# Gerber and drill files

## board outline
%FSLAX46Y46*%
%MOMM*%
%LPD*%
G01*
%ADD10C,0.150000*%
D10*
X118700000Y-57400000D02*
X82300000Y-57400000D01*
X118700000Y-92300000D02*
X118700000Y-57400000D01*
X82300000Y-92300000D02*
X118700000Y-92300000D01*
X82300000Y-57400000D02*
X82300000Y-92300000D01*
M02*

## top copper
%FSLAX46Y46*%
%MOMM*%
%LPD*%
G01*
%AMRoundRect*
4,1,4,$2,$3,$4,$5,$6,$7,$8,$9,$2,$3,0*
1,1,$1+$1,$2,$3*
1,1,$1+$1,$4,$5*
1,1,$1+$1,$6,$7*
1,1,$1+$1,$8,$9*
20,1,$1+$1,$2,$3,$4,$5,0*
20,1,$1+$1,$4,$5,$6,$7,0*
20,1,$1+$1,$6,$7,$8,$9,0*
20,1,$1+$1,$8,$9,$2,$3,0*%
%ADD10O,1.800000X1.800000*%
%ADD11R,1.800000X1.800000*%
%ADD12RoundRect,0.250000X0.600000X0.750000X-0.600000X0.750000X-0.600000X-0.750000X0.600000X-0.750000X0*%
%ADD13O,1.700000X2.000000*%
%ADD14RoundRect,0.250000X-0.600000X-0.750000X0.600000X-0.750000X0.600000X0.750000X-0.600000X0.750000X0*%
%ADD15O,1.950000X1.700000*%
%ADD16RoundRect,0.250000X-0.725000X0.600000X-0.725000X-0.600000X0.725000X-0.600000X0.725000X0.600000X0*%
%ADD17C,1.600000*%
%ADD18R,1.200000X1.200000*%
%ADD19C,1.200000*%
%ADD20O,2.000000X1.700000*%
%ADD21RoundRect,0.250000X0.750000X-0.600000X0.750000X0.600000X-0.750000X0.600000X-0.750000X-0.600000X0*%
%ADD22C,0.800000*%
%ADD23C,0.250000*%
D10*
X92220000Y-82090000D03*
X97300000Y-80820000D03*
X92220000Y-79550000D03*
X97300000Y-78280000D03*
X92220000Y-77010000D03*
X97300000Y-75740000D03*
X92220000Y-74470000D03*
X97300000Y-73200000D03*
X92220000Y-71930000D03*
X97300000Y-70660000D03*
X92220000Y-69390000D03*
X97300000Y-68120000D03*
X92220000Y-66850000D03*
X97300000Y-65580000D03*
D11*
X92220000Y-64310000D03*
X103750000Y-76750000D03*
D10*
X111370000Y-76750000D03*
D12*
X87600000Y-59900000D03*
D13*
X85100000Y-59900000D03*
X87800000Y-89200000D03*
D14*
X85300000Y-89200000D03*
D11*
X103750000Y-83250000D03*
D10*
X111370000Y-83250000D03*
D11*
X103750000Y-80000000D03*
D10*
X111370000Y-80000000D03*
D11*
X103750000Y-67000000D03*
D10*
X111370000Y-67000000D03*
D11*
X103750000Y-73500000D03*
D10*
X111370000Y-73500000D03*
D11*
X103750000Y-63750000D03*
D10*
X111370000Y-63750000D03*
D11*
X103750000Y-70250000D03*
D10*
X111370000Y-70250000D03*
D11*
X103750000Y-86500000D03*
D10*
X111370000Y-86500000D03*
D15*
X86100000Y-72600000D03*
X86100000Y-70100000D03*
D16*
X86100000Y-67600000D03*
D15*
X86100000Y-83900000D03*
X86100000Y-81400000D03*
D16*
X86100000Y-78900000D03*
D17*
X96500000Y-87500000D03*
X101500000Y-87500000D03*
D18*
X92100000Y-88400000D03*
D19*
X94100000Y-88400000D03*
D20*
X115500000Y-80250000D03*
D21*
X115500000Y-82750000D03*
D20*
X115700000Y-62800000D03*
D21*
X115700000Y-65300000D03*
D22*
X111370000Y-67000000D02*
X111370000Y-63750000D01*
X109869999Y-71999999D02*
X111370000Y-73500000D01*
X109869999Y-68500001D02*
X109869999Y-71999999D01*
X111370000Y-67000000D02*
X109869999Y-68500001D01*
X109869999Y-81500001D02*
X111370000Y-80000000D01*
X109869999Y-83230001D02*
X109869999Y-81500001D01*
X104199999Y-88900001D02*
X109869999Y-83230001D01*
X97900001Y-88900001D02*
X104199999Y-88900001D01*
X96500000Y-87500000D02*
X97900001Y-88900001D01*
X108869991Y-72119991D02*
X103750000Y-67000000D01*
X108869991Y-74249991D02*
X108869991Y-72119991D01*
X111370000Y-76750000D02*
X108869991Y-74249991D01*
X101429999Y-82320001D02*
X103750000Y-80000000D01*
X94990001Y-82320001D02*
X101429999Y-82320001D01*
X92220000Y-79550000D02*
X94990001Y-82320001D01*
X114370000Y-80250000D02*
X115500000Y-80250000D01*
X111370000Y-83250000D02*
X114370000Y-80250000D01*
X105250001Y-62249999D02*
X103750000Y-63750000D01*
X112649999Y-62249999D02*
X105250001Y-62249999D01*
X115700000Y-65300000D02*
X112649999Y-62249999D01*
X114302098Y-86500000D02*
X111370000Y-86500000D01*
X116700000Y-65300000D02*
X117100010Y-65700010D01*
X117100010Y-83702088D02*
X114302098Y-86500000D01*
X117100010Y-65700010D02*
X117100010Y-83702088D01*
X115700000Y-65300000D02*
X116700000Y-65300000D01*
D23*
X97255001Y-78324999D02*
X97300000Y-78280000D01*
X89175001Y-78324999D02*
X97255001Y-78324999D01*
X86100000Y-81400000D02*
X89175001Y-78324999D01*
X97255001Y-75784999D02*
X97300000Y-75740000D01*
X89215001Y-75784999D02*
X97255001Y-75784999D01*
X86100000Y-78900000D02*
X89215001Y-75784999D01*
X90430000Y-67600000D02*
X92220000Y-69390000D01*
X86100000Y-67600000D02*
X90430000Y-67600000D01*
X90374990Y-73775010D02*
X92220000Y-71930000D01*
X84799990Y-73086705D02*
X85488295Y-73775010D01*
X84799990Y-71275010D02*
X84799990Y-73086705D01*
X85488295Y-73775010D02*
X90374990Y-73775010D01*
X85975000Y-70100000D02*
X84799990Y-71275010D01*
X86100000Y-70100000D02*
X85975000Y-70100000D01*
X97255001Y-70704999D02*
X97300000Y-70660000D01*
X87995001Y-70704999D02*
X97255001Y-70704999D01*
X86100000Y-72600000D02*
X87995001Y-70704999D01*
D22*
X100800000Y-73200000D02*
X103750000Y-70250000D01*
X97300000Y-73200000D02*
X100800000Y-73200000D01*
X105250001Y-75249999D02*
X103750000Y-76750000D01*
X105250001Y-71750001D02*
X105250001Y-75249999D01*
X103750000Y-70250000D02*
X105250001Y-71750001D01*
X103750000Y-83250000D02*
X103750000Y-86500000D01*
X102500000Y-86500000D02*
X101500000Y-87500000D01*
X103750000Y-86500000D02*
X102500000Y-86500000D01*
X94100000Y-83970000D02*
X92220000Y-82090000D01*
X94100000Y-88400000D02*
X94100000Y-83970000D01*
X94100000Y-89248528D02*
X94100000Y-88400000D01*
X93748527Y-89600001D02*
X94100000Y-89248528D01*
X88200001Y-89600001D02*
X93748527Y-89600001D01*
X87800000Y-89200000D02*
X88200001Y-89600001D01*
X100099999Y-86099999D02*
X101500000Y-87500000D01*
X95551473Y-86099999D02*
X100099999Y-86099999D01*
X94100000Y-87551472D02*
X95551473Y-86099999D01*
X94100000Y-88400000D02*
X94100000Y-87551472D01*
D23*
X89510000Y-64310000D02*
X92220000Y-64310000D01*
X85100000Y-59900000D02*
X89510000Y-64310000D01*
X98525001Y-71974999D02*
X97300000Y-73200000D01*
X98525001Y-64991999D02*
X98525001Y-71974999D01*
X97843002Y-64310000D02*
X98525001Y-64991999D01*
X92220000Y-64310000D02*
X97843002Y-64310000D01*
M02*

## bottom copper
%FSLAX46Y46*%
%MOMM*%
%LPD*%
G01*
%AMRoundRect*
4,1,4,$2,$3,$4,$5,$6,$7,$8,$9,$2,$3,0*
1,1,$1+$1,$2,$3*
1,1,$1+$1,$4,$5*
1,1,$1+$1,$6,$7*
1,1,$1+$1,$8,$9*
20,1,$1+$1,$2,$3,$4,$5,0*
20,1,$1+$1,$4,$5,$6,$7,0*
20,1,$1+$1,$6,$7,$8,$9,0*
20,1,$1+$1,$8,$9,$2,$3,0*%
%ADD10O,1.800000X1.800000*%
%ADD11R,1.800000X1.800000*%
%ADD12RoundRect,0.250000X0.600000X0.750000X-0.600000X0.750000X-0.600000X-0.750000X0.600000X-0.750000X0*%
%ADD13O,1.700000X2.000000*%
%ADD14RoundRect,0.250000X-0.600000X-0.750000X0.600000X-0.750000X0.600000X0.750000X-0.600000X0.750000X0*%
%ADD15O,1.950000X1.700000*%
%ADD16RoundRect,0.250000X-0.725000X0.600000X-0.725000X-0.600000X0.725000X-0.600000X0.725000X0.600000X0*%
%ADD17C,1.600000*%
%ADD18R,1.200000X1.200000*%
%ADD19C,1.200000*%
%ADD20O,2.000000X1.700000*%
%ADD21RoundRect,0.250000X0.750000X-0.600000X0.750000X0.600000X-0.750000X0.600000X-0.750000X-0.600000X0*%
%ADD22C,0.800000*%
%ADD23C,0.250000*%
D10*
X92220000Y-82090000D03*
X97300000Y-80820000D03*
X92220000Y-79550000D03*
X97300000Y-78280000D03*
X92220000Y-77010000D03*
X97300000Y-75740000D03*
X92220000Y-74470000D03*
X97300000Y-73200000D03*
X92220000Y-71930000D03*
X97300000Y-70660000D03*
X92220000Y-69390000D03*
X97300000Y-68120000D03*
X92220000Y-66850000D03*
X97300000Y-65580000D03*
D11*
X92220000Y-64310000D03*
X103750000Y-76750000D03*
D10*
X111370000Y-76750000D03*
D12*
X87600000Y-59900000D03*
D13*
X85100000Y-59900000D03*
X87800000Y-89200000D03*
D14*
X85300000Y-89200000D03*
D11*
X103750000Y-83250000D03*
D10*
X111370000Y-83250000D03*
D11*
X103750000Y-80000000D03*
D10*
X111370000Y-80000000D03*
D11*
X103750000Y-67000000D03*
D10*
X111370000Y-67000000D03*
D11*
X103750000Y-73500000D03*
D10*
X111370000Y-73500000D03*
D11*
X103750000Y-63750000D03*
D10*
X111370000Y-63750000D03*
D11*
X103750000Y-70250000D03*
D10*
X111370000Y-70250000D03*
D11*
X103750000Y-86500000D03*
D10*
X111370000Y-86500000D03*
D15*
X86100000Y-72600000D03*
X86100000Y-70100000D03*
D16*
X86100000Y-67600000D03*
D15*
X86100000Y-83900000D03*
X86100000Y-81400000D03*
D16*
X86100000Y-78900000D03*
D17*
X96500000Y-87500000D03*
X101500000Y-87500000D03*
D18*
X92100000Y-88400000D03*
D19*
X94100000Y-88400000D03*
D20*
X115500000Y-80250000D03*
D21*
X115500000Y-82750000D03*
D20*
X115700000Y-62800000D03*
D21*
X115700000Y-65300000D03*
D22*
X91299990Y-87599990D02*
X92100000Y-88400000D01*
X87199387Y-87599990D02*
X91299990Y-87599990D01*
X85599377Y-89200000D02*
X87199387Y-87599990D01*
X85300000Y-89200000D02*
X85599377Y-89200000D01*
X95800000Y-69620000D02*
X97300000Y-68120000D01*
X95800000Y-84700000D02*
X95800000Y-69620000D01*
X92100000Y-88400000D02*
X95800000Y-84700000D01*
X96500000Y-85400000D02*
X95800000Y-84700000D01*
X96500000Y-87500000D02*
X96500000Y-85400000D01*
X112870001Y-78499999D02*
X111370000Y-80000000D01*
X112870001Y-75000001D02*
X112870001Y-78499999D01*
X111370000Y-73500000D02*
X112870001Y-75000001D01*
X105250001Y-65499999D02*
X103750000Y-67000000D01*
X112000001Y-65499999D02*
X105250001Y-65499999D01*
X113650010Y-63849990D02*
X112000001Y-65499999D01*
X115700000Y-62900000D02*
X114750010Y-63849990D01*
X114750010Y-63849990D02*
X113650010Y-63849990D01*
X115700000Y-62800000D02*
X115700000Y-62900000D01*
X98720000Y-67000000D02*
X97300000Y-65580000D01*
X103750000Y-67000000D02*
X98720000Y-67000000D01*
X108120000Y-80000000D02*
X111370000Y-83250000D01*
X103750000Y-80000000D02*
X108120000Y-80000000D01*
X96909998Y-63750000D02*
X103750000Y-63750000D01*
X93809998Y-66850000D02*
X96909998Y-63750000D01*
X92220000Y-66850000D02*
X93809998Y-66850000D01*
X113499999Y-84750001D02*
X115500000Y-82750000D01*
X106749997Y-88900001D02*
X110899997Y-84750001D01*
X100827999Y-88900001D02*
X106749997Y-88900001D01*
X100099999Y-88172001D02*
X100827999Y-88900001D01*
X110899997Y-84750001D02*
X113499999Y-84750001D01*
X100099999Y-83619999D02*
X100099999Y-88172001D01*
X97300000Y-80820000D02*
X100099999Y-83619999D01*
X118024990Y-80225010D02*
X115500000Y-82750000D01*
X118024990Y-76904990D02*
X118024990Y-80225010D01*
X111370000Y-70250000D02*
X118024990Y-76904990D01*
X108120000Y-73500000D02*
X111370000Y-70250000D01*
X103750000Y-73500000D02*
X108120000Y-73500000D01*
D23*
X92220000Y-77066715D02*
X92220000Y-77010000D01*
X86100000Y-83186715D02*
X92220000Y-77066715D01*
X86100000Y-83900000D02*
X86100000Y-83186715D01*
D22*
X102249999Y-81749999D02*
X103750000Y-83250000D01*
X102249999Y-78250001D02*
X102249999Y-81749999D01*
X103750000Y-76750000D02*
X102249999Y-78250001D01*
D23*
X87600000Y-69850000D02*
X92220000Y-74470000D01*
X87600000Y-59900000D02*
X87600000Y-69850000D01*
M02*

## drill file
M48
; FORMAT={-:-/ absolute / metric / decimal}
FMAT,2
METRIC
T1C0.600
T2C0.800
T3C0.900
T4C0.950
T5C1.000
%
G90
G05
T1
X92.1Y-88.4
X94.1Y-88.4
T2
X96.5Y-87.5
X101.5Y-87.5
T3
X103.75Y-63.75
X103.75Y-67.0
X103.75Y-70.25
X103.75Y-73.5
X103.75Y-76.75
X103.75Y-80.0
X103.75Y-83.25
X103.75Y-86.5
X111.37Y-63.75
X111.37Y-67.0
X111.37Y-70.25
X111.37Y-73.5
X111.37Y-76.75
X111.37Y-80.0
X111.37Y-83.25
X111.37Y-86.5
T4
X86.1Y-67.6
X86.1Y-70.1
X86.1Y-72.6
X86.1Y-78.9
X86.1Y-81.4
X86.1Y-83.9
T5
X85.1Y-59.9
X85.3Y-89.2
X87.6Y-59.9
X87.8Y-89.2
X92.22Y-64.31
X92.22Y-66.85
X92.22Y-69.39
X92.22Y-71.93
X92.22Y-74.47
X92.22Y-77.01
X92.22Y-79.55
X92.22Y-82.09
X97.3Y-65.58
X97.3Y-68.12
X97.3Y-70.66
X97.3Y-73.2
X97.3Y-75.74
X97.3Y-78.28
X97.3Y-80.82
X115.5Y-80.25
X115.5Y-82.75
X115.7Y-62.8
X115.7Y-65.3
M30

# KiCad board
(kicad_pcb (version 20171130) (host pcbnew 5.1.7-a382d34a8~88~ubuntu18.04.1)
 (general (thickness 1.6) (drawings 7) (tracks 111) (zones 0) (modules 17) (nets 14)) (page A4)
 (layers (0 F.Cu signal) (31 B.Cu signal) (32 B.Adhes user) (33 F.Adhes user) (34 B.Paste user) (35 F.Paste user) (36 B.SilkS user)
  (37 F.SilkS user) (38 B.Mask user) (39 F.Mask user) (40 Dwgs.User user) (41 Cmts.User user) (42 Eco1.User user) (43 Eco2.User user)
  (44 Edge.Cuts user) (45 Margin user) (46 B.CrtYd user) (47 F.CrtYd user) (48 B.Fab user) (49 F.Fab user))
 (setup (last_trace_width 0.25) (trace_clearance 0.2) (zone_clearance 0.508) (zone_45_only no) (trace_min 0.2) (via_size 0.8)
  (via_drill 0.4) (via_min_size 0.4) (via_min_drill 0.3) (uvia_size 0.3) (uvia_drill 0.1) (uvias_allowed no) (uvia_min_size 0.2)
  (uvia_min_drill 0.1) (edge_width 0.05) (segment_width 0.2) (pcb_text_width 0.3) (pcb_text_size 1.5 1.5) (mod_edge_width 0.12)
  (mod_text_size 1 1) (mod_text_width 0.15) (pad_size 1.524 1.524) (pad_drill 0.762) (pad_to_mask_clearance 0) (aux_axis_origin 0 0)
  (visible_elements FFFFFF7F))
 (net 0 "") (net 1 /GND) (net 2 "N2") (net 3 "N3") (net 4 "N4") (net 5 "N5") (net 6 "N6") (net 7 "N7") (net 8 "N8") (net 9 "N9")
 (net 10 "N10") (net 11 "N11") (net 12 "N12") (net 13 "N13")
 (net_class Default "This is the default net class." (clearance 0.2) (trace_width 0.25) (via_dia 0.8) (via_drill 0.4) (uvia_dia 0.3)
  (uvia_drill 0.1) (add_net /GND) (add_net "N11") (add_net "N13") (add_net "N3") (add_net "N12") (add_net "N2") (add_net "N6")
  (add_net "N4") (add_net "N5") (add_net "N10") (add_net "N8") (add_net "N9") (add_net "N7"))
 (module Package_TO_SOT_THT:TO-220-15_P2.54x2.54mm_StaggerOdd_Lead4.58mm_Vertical (layer F.Cu) (at 92.22 64.31 270)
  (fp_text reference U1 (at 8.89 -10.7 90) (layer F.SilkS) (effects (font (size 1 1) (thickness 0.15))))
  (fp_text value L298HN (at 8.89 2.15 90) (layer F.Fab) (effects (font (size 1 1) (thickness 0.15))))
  (pad 15 thru_hole oval (at 17.78 0 270) (size 1.8 1.8) (drill 1) (layers *.Cu *.Mask) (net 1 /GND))
  (pad 14 thru_hole oval (at 16.51 -5.08 270) (size 1.8 1.8) (drill 1) (layers *.Cu *.Mask) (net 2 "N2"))
  (pad 13 thru_hole oval (at 15.24 0 270) (size 1.8 1.8) (drill 1) (layers *.Cu *.Mask) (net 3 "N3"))
  (pad 12 thru_hole oval (at 13.97 -5.08 270) (size 1.8 1.8) (drill 1) (layers *.Cu *.Mask) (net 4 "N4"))
  (pad 11 thru_hole oval (at 12.7 0 270) (size 1.8 1.8) (drill 1) (layers *.Cu *.Mask) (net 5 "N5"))
  (pad 10 thru_hole oval (at 11.43 -5.08 270) (size 1.8 1.8) (drill 1) (layers *.Cu *.Mask) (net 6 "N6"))
  (pad 9 thru_hole oval (at 10.16 0 270) (size 1.8 1.8) (drill 1) (layers *.Cu *.Mask) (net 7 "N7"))
  (pad 8 thru_hole oval (at 8.89 -5.08 270) (size 1.8 1.8) (drill 1) (layers *.Cu *.Mask) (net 1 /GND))
  (pad 7 thru_hole oval (at 7.62 0 270) (size 1.8 1.8) (drill 1) (layers *.Cu *.Mask) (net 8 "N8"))
  (pad 6 thru_hole oval (at 6.35 -5.08 270) (size 1.8 1.8) (drill 1) (layers *.Cu *.Mask) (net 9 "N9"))
  (pad 5 thru_hole oval (at 5.08 0 270) (size 1.8 1.8) (drill 1) (layers *.Cu *.Mask) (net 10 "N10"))
  (pad 4 thru_hole oval (at 3.81 -5.08 270) (size 1.8 1.8) (drill 1) (layers *.Cu *.Mask) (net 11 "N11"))
  (pad 3 thru_hole oval (at 2.54 0 270) (size 1.8 1.8) (drill 1) (layers *.Cu *.Mask) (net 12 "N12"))
  (pad 2 thru_hole oval (at 1.27 -5.08 270) (size 1.8 1.8) (drill 1) (layers *.Cu *.Mask) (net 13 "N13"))
  (pad 1 thru_hole rect (at 0 0 270) (size 1.8 1.8) (drill 1) (layers *.Cu *.Mask) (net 1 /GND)))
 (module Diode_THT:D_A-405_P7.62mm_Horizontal (layer F.Cu) (at 103.75 76.75)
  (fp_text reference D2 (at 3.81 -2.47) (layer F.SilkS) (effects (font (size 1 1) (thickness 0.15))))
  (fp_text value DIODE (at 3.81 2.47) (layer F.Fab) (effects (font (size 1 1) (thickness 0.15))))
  (pad 1 thru_hole rect (at 0 0) (size 1.8 1.8) (drill 0.9) (layers *.Cu *.Mask) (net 1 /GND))
  (pad 2 thru_hole oval (at 7.62 0) (size 1.8 1.8) (drill 0.9) (layers *.Cu *.Mask) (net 13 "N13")))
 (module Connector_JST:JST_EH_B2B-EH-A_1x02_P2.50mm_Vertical (layer F.Cu) (at 87.6 59.9 180)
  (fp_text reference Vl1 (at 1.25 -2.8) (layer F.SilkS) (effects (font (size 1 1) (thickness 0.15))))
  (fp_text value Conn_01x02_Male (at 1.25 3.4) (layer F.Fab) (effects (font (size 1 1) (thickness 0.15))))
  (pad 1 thru_hole roundrect (at 0 0 180) (size 1.7 2) (drill 1) (layers *.Cu *.Mask) (roundrect_rratio 0.147059) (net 7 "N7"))
  (pad 2 thru_hole oval (at 2.5 0 180) (size 1.7 2) (drill 1) (layers *.Cu *.Mask) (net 1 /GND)))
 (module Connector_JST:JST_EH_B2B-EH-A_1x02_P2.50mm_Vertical (layer F.Cu) (at 85.3 89.2)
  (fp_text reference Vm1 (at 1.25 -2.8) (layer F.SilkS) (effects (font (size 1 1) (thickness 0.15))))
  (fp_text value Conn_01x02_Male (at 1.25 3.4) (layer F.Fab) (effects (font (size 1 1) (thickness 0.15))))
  (pad 2 thru_hole oval (at 2.5 0) (size 1.7 2) (drill 1) (layers *.Cu *.Mask) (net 1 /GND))
  (pad 1 thru_hole roundrect (at 0 0) (size 1.7 2) (drill 1) (layers *.Cu *.Mask) (roundrect_rratio 0.147059) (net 11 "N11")))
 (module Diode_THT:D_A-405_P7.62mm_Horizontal (layer F.Cu) (at 103.75 83.25)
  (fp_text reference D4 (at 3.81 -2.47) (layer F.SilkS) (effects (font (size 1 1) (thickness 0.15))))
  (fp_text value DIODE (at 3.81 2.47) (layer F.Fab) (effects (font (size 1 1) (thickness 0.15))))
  (pad 1 thru_hole rect (at 0 0) (size 1.8 1.8) (drill 0.9) (layers *.Cu *.Mask) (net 1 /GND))
  (pad 2 thru_hole oval (at 7.62 0) (size 1.8 1.8) (drill 0.9) (layers *.Cu *.Mask) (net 3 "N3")))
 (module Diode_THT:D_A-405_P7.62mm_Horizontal (layer F.Cu) (at 103.75 80)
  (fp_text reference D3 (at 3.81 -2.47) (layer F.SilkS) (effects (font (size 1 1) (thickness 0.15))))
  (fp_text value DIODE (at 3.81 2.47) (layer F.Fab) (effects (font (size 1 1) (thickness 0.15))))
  (pad 1 thru_hole rect (at 0 0) (size 1.8 1.8) (drill 0.9) (layers *.Cu *.Mask) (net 3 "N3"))
  (pad 2 thru_hole oval (at 7.62 0) (size 1.8 1.8) (drill 0.9) (layers *.Cu *.Mask) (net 11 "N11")))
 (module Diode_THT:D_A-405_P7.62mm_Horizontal (layer F.Cu) (at 103.75 67)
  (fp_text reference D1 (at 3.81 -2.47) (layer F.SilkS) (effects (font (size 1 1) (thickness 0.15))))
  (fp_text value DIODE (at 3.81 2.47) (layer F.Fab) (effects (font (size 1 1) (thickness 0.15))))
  (pad 1 thru_hole rect (at 0 0) (size 1.8 1.8) (drill 0.9) (layers *.Cu *.Mask) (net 13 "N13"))
  (pad 2 thru_hole oval (at 7.62 0) (size 1.8 1.8) (drill 0.9) (layers *.Cu *.Mask) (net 11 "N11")))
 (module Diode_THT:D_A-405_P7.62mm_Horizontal (layer F.Cu) (at 103.75 73.5)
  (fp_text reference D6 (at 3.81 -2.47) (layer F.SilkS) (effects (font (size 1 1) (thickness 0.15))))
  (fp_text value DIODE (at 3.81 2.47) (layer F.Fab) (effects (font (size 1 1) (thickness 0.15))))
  (pad 1 thru_hole rect (at 0 0) (size 1.8 1.8) (drill 0.9) (layers *.Cu *.Mask) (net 2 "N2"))
  (pad 2 thru_hole oval (at 7.62 0) (size 1.8 1.8) (drill 0.9) (layers *.Cu *.Mask) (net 11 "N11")))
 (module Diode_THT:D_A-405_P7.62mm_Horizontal (layer F.Cu) (at 103.75 63.75)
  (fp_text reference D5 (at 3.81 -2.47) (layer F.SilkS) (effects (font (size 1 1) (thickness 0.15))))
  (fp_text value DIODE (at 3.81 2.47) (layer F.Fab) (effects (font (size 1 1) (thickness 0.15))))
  (pad 1 thru_hole rect (at 0 0) (size 1.8 1.8) (drill 0.9) (layers *.Cu *.Mask) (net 12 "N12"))
  (pad 2 thru_hole oval (at 7.62 0) (size 1.8 1.8) (drill 0.9) (layers *.Cu *.Mask) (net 11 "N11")))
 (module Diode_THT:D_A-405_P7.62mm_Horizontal (layer F.Cu) (at 103.75 70.25)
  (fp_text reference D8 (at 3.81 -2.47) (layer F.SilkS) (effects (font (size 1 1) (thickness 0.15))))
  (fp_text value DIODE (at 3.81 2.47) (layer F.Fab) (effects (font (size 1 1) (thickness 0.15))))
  (pad 1 thru_hole rect (at 0 0) (size 1.8 1.8) (drill 0.9) (layers *.Cu *.Mask) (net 1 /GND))
  (pad 2 thru_hole oval (at 7.62 0) (size 1.8 1.8) (drill 0.9) (layers *.Cu *.Mask) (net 2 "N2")))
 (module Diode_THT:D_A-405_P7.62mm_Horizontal (layer F.Cu) (at 103.75 86.5)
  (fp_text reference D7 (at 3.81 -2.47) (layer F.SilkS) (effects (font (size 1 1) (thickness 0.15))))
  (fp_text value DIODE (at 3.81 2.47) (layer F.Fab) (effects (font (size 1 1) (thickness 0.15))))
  (pad 1 thru_hole rect (at 0 0) (size 1.8 1.8) (drill 0.9) (layers *.Cu *.Mask) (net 1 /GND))
  (pad 2 thru_hole oval (at 7.62 0) (size 1.8 1.8) (drill 0.9) (layers *.Cu *.Mask) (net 12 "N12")))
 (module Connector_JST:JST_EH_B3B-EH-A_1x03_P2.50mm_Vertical (layer F.Cu) (at 86.1 67.6 270)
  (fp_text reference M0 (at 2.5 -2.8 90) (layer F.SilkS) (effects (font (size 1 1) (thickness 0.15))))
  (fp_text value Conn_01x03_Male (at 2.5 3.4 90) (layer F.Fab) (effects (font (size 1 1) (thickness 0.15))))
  (pad 3 thru_hole oval (at 5 0 270) (size 1.7 1.95) (drill 0.95) (layers *.Cu *.Mask) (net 9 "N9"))
  (pad 2 thru_hole oval (at 2.5 0 270) (size 1.7 1.95) (drill 0.95) (layers *.Cu *.Mask) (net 8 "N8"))
  (pad 1 thru_hole roundrect (at 0 0 270) (size 1.7 1.95) (drill 0.95) (layers *.Cu *.Mask) (roundrect_rratio 0.147059) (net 10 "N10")))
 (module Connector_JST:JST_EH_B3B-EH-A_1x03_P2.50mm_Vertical (layer F.Cu) (at 86.1 78.9 270)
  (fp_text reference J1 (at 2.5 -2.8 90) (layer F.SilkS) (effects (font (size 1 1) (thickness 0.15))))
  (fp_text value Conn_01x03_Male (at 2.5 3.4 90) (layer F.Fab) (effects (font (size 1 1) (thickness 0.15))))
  (pad 3 thru_hole oval (at 5 0 270) (size 1.7 1.95) (drill 0.95) (layers *.Cu *.Mask) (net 5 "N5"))
  (pad 2 thru_hole oval (at 2.5 0 270) (size 1.7 1.95) (drill 0.95) (layers *.Cu *.Mask) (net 4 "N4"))
  (pad 1 thru_hole roundrect (at 0 0 270) (size 1.7 1.95) (drill 0.95) (layers *.Cu *.Mask) (roundrect_rratio 0.147059) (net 6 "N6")))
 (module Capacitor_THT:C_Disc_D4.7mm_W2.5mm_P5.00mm (layer F.Cu) (at 96.5 87.5)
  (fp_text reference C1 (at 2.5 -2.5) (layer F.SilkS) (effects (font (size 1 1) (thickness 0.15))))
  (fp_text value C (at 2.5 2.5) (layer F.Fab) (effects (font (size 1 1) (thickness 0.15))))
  (pad 1 thru_hole circle (at 0 0) (size 1.6 1.6) (drill 0.8) (layers *.Cu *.Mask) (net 11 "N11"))
  (pad 2 thru_hole circle (at 5 0) (size 1.6 1.6) (drill 0.8) (layers *.Cu *.Mask) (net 1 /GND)))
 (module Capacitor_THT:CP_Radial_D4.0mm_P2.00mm (layer F.Cu) (at 92.1 88.4)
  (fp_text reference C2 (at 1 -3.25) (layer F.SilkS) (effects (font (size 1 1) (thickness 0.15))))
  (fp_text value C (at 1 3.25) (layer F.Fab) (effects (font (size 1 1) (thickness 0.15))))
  (pad 1 thru_hole rect (at 0 0) (size 1.2 1.2) (drill 0.6) (layers *.Cu *.Mask) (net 11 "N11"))
  (pad 2 thru_hole circle (at 2 0) (size 1.2 1.2) (drill 0.6) (layers *.Cu *.Mask) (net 1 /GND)))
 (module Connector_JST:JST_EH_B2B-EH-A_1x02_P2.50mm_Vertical (layer F.Cu) (at 115.5 82.75 90)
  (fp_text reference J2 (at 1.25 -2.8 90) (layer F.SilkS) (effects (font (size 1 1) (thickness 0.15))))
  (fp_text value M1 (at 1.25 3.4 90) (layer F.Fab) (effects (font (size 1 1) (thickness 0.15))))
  (pad 2 thru_hole oval (at 2.5 0 90) (size 1.7 2) (drill 1) (layers *.Cu *.Mask) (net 3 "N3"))
  (pad 1 thru_hole roundrect (at 0 0 90) (size 1.7 2) (drill 1) (layers *.Cu *.Mask) (roundrect_rratio 0.147059) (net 2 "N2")))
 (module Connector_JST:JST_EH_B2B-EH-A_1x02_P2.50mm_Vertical (layer F.Cu) (at 115.7 65.3 90)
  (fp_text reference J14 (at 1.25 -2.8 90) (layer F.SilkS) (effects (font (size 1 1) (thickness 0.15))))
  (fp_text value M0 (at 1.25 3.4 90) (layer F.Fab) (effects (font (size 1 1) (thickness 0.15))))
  (pad 2 thru_hole oval (at 2.5 0 90) (size 1.7 2) (drill 1) (layers *.Cu *.Mask) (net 13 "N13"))
  (pad 1 thru_hole roundrect (at 0 0 90) (size 1.7 2) (drill 1) (layers *.Cu *.Mask) (roundrect_rratio 0.147059) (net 12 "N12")))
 (gr_line (start 118.7 57.4) (end 82.3 57.4) (layer Edge.Cuts) (width 0.15))
 (gr_line (start 118.7 92.3) (end 118.7 57.4) (layer Edge.Cuts) (width 0.15))
 (gr_line (start 82.3 92.3) (end 118.7 92.3) (layer Edge.Cuts) (width 0.15))
 (gr_line (start 82.3 57.4) (end 82.3 92.3) (layer Edge.Cuts) (width 0.15))
 (segment (start 91.29999 87.59999) (end 92.1 88.4) (width 0.8) (layer B.Cu) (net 11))
 (segment (start 87.199387 87.59999) (end 91.29999 87.59999) (width 0.8) (layer B.Cu) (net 11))
 (segment (start 85.599377 89.2) (end 87.199387 87.59999) (width 0.8) (layer B.Cu) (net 11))
 (segment (start 85.3 89.2) (end 85.599377 89.2) (width 0.8) (layer B.Cu) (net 11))
 (segment (start 95.8 69.62) (end 97.3 68.12) (width 0.8) (layer B.Cu) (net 11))
 (segment (start 95.8 84.7) (end 95.8 69.62) (width 0.8) (layer B.Cu) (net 11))
 (segment (start 92.1 88.4) (end 95.8 84.7) (width 0.8) (layer B.Cu) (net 11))
 (segment (start 96.5 85.4) (end 95.8 84.7) (width 0.8) (layer B.Cu) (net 11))
 (segment (start 96.5 87.5) (end 96.5 85.4) (width 0.8) (layer B.Cu) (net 11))
 (segment (start 111.37 67) (end 111.37 63.75) (width 0.8) (layer F.Cu) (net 11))
 (segment (start 109.869999 71.999999) (end 111.37 73.5) (width 0.8) (layer F.Cu) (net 11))
 (segment (start 109.869999 68.500001) (end 109.869999 71.999999) (width 0.8) (layer F.Cu) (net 11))
 (segment (start 111.37 67) (end 109.869999 68.500001) (width 0.8) (layer F.Cu) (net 11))
 (segment (start 112.870001 78.499999) (end 111.37 80) (width 0.8) (layer B.Cu) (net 11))
 (segment (start 112.870001 75.000001) (end 112.870001 78.499999) (width 0.8) (layer B.Cu) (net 11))
 (segment (start 111.37 73.5) (end 112.870001 75.000001) (width 0.8) (layer B.Cu) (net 11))
 (segment (start 109.869999 81.500001) (end 111.37 80) (width 0.8) (layer F.Cu) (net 11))
 (segment (start 109.869999 83.230001) (end 109.869999 81.500001) (width 0.8) (layer F.Cu) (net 11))
 (segment (start 104.199999 88.900001) (end 109.869999 83.230001) (width 0.8) (layer F.Cu) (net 11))
 (segment (start 97.900001 88.900001) (end 104.199999 88.900001) (width 0.8) (layer F.Cu) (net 11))
 (segment (start 96.5 87.5) (end 97.900001 88.900001) (width 0.8) (layer F.Cu) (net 11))
 (segment (start 105.250001 65.499999) (end 103.75 67) (width 0.8) (layer B.Cu) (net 13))
 (segment (start 112.000001 65.499999) (end 105.250001 65.499999) (width 0.8) (layer B.Cu) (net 13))
 (segment (start 113.65001 63.84999) (end 112.000001 65.499999) (width 0.8) (layer B.Cu) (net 13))
 (segment (start 115.7 62.9) (end 114.75001 63.84999) (width 0.8) (layer B.Cu) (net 13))
 (segment (start 114.75001 63.84999) (end 113.65001 63.84999) (width 0.8) (layer B.Cu) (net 13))
 (segment (start 115.7 62.8) (end 115.7 62.9) (width 0.8) (layer B.Cu) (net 13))
 (segment (start 98.72 67) (end 97.3 65.58) (width 0.8) (layer B.Cu) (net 13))
 (segment (start 103.75 67) (end 98.72 67) (width 0.8) (layer B.Cu) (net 13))
 (segment (start 108.869991 72.119991) (end 103.75 67) (width 0.8) (layer F.Cu) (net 13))
 (segment (start 108.869991 74.249991) (end 108.869991 72.119991) (width 0.8) (layer F.Cu) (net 13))
 (segment (start 111.37 76.75) (end 108.869991 74.249991) (width 0.8) (layer F.Cu) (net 13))
 (segment (start 101.429999 82.320001) (end 103.75 80) (width 0.8) (layer F.Cu) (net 3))
 (segment (start 94.990001 82.320001) (end 101.429999 82.320001) (width 0.8) (layer F.Cu) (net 3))
 (segment (start 92.22 79.55) (end 94.990001 82.320001) (width 0.8) (layer F.Cu) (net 3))
 (segment (start 114.37 80.25) (end 115.5 80.25) (width 0.8) (layer F.Cu) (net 3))
 (segment (start 111.37 83.25) (end 114.37 80.25) (width 0.8) (layer F.Cu) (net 3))
 (segment (start 108.12 80) (end 111.37 83.25) (width 0.8) (layer B.Cu) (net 3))
 (segment (start 103.75 80) (end 108.12 80) (width 0.8) (layer B.Cu) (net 3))
 (segment (start 105.250001 62.249999) (end 103.75 63.75) (width 0.8) (layer F.Cu) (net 12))
 (segment (start 112.649999 62.249999) (end 105.250001 62.249999) (width 0.8) (layer F.Cu) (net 12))
 (segment (start 115.7 65.3) (end 112.649999 62.249999) (width 0.8) (layer F.Cu) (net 12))
 (segment (start 114.302098 86.5) (end 111.37 86.5) (width 0.8) (layer F.Cu) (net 12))
 (segment (start 116.7 65.3) (end 117.10001 65.70001) (width 0.8) (layer F.Cu) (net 12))
 (segment (start 117.10001 83.702088) (end 114.302098 86.5) (width 0.8) (layer F.Cu) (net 12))
 (segment (start 117.10001 65.70001) (end 117.10001 83.702088) (width 0.8) (layer F.Cu) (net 12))
 (segment (start 115.7 65.3) (end 116.7 65.3) (width 0.8) (layer F.Cu) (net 12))
 (segment (start 96.909998 63.75) (end 103.75 63.75) (width 0.8) (layer B.Cu) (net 12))
 (segment (start 93.809998 66.85) (end 96.909998 63.75) (width 0.8) (layer B.Cu) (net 12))
 (segment (start 92.22 66.85) (end 93.809998 66.85) (width 0.8) (layer B.Cu) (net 12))
 (segment (start 113.499999 84.750001) (end 115.5 82.75) (width 0.8) (layer B.Cu) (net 2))
 (segment (start 106.749997 88.900001) (end 110.899997 84.750001) (width 0.8) (layer B.Cu) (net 2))
 (segment (start 100.827999 88.900001) (end 106.749997 88.900001) (width 0.8) (layer B.Cu) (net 2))
 (segment (start 100.099999 88.172001) (end 100.827999 88.900001) (width 0.8) (layer B.Cu) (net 2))
 (segment (start 110.899997 84.750001) (end 113.499999 84.750001) (width 0.8) (layer B.Cu) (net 2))
 (segment (start 100.099999 83.619999) (end 100.099999 88.172001) (width 0.8) (layer B.Cu) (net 2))
 (segment (start 97.3 80.82) (end 100.099999 83.619999) (width 0.8) (layer B.Cu) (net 2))
 (segment (start 118.02499 80.22501) (end 115.5 82.75) (width 0.8) (layer B.Cu) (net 2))
 (segment (start 118.02499 76.90499) (end 118.02499 80.22501) (width 0.8) (layer B.Cu) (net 2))
 (segment (start 111.37 70.25) (end 118.02499 76.90499) (width 0.8) (layer B.Cu) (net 2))
 (segment (start 108.12 73.5) (end 111.37 70.25) (width 0.8) (layer B.Cu) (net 2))
 (segment (start 103.75 73.5) (end 108.12 73.5) (width 0.8) (layer B.Cu) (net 2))
 (segment (start 92.22 77.066715) (end 92.22 77.01) (width 0.25) (layer B.Cu) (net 5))
 (segment (start 86.1 83.186715) (end 92.22 77.066715) (width 0.25) (layer B.Cu) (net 5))
 (segment (start 86.1 83.9) (end 86.1 83.186715) (width 0.25) (layer B.Cu) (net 5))
 (segment (start 97.255001 78.324999) (end 97.3 78.28) (width 0.25) (layer F.Cu) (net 4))
 (segment (start 89.175001 78.324999) (end 97.255001 78.324999) (width 0.25) (layer F.Cu) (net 4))
 (segment (start 86.1 81.4) (end 89.175001 78.324999) (width 0.25) (layer F.Cu) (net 4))
 (segment (start 97.255001 75.784999) (end 97.3 75.74) (width 0.25) (layer F.Cu) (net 6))
 (segment (start 89.215001 75.784999) (end 97.255001 75.784999) (width 0.25) (layer F.Cu) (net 6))
 (segment (start 86.1 78.9) (end 89.215001 75.784999) (width 0.25) (layer F.Cu) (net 6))
 (segment (start 90.43 67.6) (end 92.22 69.39) (width 0.25) (layer F.Cu) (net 10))
 (segment (start 86.1 67.6) (end 90.43 67.6) (width 0.25) (layer F.Cu) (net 10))
 (segment (start 90.37499 73.77501) (end 92.22 71.93) (width 0.25) (layer F.Cu) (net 8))
 (segment (start 84.79999 73.086705) (end 85.488295 73.77501) (width 0.25) (layer F.Cu) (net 8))
 (segment (start 84.79999 71.27501) (end 84.79999 73.086705) (width 0.25) (layer F.Cu) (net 8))
 (segment (start 85.488295 73.77501) (end 90.37499 73.77501) (width 0.25) (layer F.Cu) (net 8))
 (segment (start 85.975 70.1) (end 84.79999 71.27501) (width 0.25) (layer F.Cu) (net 8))
 (segment (start 86.1 70.1) (end 85.975 70.1) (width 0.25) (layer F.Cu) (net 8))
 (segment (start 97.255001 70.704999) (end 97.3 70.66) (width 0.25) (layer F.Cu) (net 9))
 (segment (start 87.995001 70.704999) (end 97.255001 70.704999) (width 0.25) (layer F.Cu) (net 9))
 (segment (start 86.1 72.6) (end 87.995001 70.704999) (width 0.25) (layer F.Cu) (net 9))
 (segment (start 100.8 73.2) (end 103.75 70.25) (width 0.8) (layer F.Cu) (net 1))
 (segment (start 97.3 73.2) (end 100.8 73.2) (width 0.8) (layer F.Cu) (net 1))
 (segment (start 105.250001 75.249999) (end 103.75 76.75) (width 0.8) (layer F.Cu) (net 1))
 (segment (start 105.250001 71.750001) (end 105.250001 75.249999) (width 0.8) (layer F.Cu) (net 1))
 (segment (start 103.75 70.25) (end 105.250001 71.750001) (width 0.8) (layer F.Cu) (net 1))
 (segment (start 103.75 83.25) (end 103.75 86.5) (width 0.8) (layer F.Cu) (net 1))
 (segment (start 102.5 86.5) (end 101.5 87.5) (width 0.8) (layer F.Cu) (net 1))
 (segment (start 103.75 86.5) (end 102.5 86.5) (width 0.8) (layer F.Cu) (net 1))
 (segment (start 94.1 83.97) (end 92.22 82.09) (width 0.8) (layer F.Cu) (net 1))
 (segment (start 94.1 88.4) (end 94.1 83.97) (width 0.8) (layer F.Cu) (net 1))
 (segment (start 94.1 89.248528) (end 94.1 88.4) (width 0.8) (layer F.Cu) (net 1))
 (segment (start 93.748527 89.600001) (end 94.1 89.248528) (width 0.8) (layer F.Cu) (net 1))
 (segment (start 88.200001 89.600001) (end 93.748527 89.600001) (width 0.8) (layer F.Cu) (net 1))
 (segment (start 87.8 89.2) (end 88.200001 89.600001) (width 0.8) (layer F.Cu) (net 1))
 (segment (start 102.249999 81.749999) (end 103.75 83.25) (width 0.8) (layer B.Cu) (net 1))
 (segment (start 102.249999 78.250001) (end 102.249999 81.749999) (width 0.8) (layer B.Cu) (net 1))
 (segment (start 103.75 76.75) (end 102.249999 78.250001) (width 0.8) (layer B.Cu) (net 1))
 (segment (start 100.099999 86.099999) (end 101.5 87.5) (width 0.8) (layer F.Cu) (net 1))
 (segment (start 95.551473 86.099999) (end 100.099999 86.099999) (width 0.8) (layer F.Cu) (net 1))
 (segment (start 94.1 87.551472) (end 95.551473 86.099999) (width 0.8) (layer F.Cu) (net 1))
 (segment (start 94.1 88.4) (end 94.1 87.551472) (width 0.8) (layer F.Cu) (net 1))
 (segment (start 89.51 64.31) (end 92.22 64.31) (width 0.25) (layer F.Cu) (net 1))
 (segment (start 85.1 59.9) (end 89.51 64.31) (width 0.25) (layer F.Cu) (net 1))
 (segment (start 98.525001 71.974999) (end 97.3 73.2) (width 0.25) (layer F.Cu) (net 1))
 (segment (start 98.525001 64.991999) (end 98.525001 71.974999) (width 0.25) (layer F.Cu) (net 1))
 (segment (start 97.843002 64.31) (end 98.525001 64.991999) (width 0.25) (layer F.Cu) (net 1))
 (segment (start 92.22 64.31) (end 97.843002 64.31) (width 0.25) (layer F.Cu) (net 1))
 (segment (start 87.6 69.85) (end 92.22 74.47) (width 0.25) (layer B.Cu) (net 7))
 (segment (start 87.6 59.9) (end 87.6 69.85) (width 0.25) (layer B.Cu) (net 7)))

